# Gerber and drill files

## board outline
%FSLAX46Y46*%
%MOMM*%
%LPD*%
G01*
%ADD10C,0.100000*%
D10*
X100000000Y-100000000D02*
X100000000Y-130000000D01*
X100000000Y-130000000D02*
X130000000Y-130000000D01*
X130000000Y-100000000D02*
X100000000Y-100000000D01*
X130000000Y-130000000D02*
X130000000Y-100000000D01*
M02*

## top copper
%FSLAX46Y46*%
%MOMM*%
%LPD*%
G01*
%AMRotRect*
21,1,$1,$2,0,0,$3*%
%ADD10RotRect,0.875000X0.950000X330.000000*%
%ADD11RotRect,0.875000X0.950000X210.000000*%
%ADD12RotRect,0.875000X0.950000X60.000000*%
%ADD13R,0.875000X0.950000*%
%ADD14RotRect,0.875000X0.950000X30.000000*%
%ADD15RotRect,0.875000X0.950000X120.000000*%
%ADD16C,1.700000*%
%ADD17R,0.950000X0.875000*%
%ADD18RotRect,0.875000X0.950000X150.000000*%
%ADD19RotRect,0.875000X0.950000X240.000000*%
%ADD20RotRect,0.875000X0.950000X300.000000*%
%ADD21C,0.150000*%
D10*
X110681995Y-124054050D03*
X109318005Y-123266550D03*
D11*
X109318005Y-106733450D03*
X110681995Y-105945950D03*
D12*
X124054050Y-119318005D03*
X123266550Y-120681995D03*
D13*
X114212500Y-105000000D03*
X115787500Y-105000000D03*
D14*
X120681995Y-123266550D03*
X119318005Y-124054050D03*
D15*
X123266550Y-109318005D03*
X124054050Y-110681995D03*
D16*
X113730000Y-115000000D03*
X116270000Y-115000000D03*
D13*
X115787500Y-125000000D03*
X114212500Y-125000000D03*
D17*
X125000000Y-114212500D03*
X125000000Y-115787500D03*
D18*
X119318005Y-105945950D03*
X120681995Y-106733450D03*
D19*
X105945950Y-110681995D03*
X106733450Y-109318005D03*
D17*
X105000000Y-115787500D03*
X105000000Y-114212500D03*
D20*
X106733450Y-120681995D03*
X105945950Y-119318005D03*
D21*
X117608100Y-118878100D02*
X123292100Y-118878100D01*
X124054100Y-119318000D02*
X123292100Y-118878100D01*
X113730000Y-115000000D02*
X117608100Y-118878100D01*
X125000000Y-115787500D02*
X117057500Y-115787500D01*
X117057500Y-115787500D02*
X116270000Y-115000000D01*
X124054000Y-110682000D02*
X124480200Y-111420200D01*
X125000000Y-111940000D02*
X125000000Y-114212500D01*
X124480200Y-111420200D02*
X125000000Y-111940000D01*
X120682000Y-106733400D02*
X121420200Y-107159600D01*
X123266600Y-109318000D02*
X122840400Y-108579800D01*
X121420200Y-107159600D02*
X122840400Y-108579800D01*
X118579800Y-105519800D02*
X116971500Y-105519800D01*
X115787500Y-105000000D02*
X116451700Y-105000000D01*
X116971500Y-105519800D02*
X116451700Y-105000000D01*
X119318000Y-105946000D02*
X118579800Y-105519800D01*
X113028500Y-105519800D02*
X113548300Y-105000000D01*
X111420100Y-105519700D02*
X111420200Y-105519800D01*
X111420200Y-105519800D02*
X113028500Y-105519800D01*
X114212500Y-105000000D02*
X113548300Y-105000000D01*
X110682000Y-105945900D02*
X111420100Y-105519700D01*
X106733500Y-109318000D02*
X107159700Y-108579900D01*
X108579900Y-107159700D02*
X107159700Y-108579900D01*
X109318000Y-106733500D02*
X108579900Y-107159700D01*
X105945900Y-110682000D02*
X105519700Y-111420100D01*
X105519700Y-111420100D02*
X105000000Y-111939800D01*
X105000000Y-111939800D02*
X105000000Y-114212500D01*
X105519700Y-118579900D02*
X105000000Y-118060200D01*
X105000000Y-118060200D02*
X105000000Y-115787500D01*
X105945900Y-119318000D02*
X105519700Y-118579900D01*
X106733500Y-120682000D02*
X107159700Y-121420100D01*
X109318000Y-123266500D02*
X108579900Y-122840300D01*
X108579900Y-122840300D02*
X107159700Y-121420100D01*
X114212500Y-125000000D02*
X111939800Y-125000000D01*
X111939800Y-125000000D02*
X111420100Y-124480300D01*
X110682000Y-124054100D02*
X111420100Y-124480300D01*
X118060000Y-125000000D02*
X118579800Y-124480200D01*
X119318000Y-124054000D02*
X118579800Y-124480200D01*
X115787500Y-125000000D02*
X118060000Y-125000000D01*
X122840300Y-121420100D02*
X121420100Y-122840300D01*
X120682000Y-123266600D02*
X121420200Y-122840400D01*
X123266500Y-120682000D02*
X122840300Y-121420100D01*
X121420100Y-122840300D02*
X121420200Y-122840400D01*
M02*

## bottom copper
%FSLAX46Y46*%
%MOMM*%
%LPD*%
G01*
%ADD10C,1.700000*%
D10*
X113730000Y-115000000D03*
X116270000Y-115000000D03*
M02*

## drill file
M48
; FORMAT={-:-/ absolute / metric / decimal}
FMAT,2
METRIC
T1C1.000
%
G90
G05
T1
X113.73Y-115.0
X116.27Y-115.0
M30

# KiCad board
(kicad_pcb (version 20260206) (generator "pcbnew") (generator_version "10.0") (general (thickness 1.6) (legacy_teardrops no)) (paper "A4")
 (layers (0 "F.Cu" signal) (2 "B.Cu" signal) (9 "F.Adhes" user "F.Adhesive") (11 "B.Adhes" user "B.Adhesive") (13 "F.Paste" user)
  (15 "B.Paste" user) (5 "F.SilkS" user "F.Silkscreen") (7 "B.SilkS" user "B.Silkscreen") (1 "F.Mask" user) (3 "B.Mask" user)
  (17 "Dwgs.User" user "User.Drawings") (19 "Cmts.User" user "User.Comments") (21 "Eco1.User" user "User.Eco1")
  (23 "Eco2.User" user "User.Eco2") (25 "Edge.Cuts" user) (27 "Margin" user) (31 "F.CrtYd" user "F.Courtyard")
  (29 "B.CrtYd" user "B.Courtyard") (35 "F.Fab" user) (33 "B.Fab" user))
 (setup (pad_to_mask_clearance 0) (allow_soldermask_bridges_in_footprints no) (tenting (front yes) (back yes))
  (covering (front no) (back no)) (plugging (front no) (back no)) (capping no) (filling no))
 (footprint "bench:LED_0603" (layer "F.Cu") (at 110 123.6603 -30)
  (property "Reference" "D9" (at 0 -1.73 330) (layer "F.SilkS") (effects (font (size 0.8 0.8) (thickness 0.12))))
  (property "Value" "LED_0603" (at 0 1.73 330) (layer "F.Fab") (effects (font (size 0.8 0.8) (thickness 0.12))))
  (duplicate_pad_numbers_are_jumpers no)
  (pad "A" smd rect (at 0.7875 0 330) (size 0.875 0.95) (layers "F.Cu" "F.Mask" "F.Paste") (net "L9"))
  (pad "K" smd rect (at -0.7875 0 330) (size 0.875 0.95) (layers "F.Cu" "F.Mask" "F.Paste") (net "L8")))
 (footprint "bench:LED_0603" (layer "F.Cu") (at 110 106.3397 -150)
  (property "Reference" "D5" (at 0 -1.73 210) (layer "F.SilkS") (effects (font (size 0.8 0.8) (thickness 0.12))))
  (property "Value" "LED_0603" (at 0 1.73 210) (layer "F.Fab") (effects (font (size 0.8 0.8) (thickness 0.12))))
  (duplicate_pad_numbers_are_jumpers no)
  (pad "A" smd rect (at 0.7875 0 210) (size 0.875 0.95) (layers "F.Cu" "F.Mask" "F.Paste") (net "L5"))
  (pad "K" smd rect (at -0.7875 0 210) (size 0.875 0.95) (layers "F.Cu" "F.Mask" "F.Paste") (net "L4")))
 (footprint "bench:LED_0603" (layer "F.Cu") (at 123.6603 120 60)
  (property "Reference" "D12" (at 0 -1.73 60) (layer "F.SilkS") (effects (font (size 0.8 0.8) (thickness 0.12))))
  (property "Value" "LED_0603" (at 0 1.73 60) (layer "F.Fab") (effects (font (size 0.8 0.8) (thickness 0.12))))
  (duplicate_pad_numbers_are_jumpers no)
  (pad "A" smd rect (at 0.7875 0 60) (size 0.875 0.95) (layers "F.Cu" "F.Mask" "F.Paste") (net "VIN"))
  (pad "K" smd rect (at -0.7875 0 60) (size 0.875 0.95) (layers "F.Cu" "F.Mask" "F.Paste") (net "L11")))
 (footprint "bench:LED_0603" (layer "F.Cu") (at 115 105 180)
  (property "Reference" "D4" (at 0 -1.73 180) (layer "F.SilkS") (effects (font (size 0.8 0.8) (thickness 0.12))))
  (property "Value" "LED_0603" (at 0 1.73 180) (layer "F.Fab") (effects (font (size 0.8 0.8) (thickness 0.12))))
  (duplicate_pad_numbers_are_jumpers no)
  (pad "A" smd rect (at 0.7875 0 180) (size 0.875 0.95) (layers "F.Cu" "F.Mask" "F.Paste") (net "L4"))
  (pad "K" smd rect (at -0.7875 0 180) (size 0.875 0.95) (layers "F.Cu" "F.Mask" "F.Paste") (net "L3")))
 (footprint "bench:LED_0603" (layer "F.Cu") (at 120 123.6603 30)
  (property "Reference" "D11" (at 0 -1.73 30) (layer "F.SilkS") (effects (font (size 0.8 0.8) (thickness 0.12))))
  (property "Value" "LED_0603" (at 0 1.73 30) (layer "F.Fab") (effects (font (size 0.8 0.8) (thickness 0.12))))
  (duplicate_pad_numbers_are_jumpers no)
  (pad "A" smd rect (at 0.7875 0 30) (size 0.875 0.95) (layers "F.Cu" "F.Mask" "F.Paste") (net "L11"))
  (pad "K" smd rect (at -0.7875 0 30) (size 0.875 0.95) (layers "F.Cu" "F.Mask" "F.Paste") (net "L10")))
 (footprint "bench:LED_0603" (layer "F.Cu") (at 123.6603 110 120)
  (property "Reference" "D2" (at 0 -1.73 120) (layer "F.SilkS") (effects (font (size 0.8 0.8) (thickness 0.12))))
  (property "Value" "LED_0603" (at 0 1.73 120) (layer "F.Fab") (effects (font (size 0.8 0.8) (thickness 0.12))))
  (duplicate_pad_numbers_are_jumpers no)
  (pad "A" smd rect (at 0.7875 0 120) (size 0.875 0.95) (layers "F.Cu" "F.Mask" "F.Paste") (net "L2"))
  (pad "K" smd rect (at -0.7875 0 120) (size 0.875 0.95) (layers "F.Cu" "F.Mask" "F.Paste") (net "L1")))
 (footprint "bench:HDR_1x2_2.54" (layer "F.Cu") (at 113.73 115)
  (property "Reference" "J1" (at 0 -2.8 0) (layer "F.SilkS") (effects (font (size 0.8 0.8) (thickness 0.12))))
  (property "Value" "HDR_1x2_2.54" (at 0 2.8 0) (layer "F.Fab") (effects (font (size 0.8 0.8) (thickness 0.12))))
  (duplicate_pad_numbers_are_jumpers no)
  (pad "1" thru_hole circle (at 0 0) (size 1.7 1.7) (drill 1) (layers "*.Cu" "*.Mask") (remove_unused_layers no) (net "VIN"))
  (pad "2" thru_hole circle (at 2.54 0) (size 1.7 1.7) (drill 1) (layers "*.Cu" "*.Mask") (remove_unused_layers no) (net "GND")))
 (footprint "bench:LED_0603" (layer "F.Cu") (at 115 125)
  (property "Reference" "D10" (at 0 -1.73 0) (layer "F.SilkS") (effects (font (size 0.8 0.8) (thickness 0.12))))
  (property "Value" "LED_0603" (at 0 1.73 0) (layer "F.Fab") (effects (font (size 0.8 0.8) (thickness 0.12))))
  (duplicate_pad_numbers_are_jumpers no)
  (pad "A" smd rect (at 0.7875 0) (size 0.875 0.95) (layers "F.Cu" "F.Mask" "F.Paste") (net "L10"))
  (pad "K" smd rect (at -0.7875 0) (size 0.875 0.95) (layers "F.Cu" "F.Mask" "F.Paste") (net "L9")))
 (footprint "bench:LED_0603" (layer "F.Cu") (at 125 115 90)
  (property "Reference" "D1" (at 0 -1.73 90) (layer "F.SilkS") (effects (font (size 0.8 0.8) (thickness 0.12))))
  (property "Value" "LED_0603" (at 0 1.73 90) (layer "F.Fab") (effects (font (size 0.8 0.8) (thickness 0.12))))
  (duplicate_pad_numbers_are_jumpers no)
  (pad "A" smd rect (at 0.7875 0 90) (size 0.875 0.95) (layers "F.Cu" "F.Mask" "F.Paste") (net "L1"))
  (pad "K" smd rect (at -0.7875 0 90) (size 0.875 0.95) (layers "F.Cu" "F.Mask" "F.Paste") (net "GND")))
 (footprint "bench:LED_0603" (layer "F.Cu") (at 120 106.3397 150)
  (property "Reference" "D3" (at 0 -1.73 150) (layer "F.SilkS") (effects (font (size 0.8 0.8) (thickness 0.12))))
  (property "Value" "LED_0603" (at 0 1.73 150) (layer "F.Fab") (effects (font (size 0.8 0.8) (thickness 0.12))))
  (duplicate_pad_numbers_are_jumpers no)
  (pad "A" smd rect (at 0.7875 0 150) (size 0.875 0.95) (layers "F.Cu" "F.Mask" "F.Paste") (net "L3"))
  (pad "K" smd rect (at -0.7875 0 150) (size 0.875 0.95) (layers "F.Cu" "F.Mask" "F.Paste") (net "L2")))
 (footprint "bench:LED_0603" (layer "F.Cu") (at 106.3397 110 -120)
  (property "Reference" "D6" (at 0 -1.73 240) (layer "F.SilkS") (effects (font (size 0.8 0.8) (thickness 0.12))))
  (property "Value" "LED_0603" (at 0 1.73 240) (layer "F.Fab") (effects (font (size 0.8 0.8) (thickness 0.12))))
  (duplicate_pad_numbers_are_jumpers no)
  (pad "A" smd rect (at 0.7875 0 240) (size 0.875 0.95) (layers "F.Cu" "F.Mask" "F.Paste") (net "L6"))
  (pad "K" smd rect (at -0.7875 0 240) (size 0.875 0.95) (layers "F.Cu" "F.Mask" "F.Paste") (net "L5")))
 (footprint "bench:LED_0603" (layer "F.Cu") (at 105 115 -90)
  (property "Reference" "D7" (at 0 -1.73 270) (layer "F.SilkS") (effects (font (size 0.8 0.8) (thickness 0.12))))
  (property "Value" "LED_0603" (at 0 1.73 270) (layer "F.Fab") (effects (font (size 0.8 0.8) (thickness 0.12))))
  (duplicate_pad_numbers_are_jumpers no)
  (pad "A" smd rect (at 0.7875 0 270) (size 0.875 0.95) (layers "F.Cu" "F.Mask" "F.Paste") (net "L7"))
  (pad "K" smd rect (at -0.7875 0 270) (size 0.875 0.95) (layers "F.Cu" "F.Mask" "F.Paste") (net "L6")))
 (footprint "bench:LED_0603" (layer "F.Cu") (at 106.3397 120 -60)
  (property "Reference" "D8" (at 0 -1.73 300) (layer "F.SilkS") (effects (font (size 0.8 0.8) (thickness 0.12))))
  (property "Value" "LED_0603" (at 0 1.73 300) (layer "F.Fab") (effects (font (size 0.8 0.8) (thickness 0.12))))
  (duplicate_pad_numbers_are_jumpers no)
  (pad "A" smd rect (at 0.7875 0 300) (size 0.875 0.95) (layers "F.Cu" "F.Mask" "F.Paste") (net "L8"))
  (pad "K" smd rect (at -0.7875 0 300) (size 0.875 0.95) (layers "F.Cu" "F.Mask" "F.Paste") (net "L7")))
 (gr_line (start 100 100) (end 100 130) (stroke (width 0.1) (type solid)) (layer "Edge.Cuts"))
 (gr_line (start 100 130) (end 130 130) (stroke (width 0.1) (type solid)) (layer "Edge.Cuts"))
 (gr_line (start 130 100) (end 100 100) (stroke (width 0.1) (type solid)) (layer "Edge.Cuts"))
 (gr_line (start 130 130) (end 130 100) (stroke (width 0.1) (type solid)) (layer "Edge.Cuts"))
 (segment (start 117.6081 118.8781) (end 123.2921 118.8781) (width 0.15) (layer "F.Cu") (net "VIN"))
 (segment (start 124.0541 119.318) (end 123.2921 118.8781) (width 0.15) (layer "F.Cu") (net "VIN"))
 (segment (start 113.73 115) (end 117.6081 118.8781) (width 0.15) (layer "F.Cu") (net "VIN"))
 (segment (start 125 115.7875) (end 117.0575 115.7875) (width 0.15) (layer "F.Cu") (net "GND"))
 (segment (start 117.0575 115.7875) (end 116.27 115) (width 0.15) (layer "F.Cu") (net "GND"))
 (segment (start 124.054 110.682) (end 124.4802 111.4202) (width 0.15) (layer "F.Cu") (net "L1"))
 (segment (start 125 111.94) (end 125 114.2125) (width 0.15) (layer "F.Cu") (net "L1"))
 (segment (start 124.4802 111.4202) (end 125 111.94) (width 0.15) (layer "F.Cu") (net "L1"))
 (segment (start 120.682 106.7334) (end 121.4202 107.1596) (width 0.15) (layer "F.Cu") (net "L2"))
 (segment (start 123.2666 109.318) (end 122.8404 108.5798) (width 0.15) (layer "F.Cu") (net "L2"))
 (segment (start 121.4202 107.1596) (end 122.8404 108.5798) (width 0.15) (layer "F.Cu") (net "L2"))
 (segment (start 118.5798 105.5198) (end 116.9715 105.5198) (width 0.15) (layer "F.Cu") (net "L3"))
 (segment (start 115.7875 105) (end 116.4517 105) (width 0.15) (layer "F.Cu") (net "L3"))
 (segment (start 116.9715 105.5198) (end 116.4517 105) (width 0.15) (layer "F.Cu") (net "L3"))
 (segment (start 119.318 105.946) (end 118.5798 105.5198) (width 0.15) (layer "F.Cu") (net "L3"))
 (segment (start 113.0285 105.5198) (end 113.5483 105) (width 0.15) (layer "F.Cu") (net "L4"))
 (segment (start 111.4201 105.5197) (end 111.4202 105.5198) (width 0.15) (layer "F.Cu") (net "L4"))
 (segment (start 111.4202 105.5198) (end 113.0285 105.5198) (width 0.15) (layer "F.Cu") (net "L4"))
 (segment (start 114.2125 105) (end 113.5483 105) (width 0.15) (layer "F.Cu") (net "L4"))
 (segment (start 110.682 105.9459) (end 111.4201 105.5197) (width 0.15) (layer "F.Cu") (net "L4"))
 (segment (start 106.7335 109.318) (end 107.1597 108.5799) (width 0.15) (layer "F.Cu") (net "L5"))
 (segment (start 108.5799 107.1597) (end 107.1597 108.5799) (width 0.15) (layer "F.Cu") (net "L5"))
 (segment (start 109.318 106.7335) (end 108.5799 107.1597) (width 0.15) (layer "F.Cu") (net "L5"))
 (segment (start 105.9459 110.682) (end 105.5197 111.4201) (width 0.15) (layer "F.Cu") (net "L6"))
 (segment (start 105.5197 111.4201) (end 105 111.9398) (width 0.15) (layer "F.Cu") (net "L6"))
 (segment (start 105 111.9398) (end 105 114.2125) (width 0.15) (layer "F.Cu") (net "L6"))
 (segment (start 105.5197 118.5799) (end 105 118.0602) (width 0.15) (layer "F.Cu") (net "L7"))
 (segment (start 105 118.0602) (end 105 115.7875) (width 0.15) (layer "F.Cu") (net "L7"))
 (segment (start 105.9459 119.318) (end 105.5197 118.5799) (width 0.15) (layer "F.Cu") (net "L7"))
 (segment (start 106.7335 120.682) (end 107.1597 121.4201) (width 0.15) (layer "F.Cu") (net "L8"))
 (segment (start 109.318 123.2665) (end 108.5799 122.8403) (width 0.15) (layer "F.Cu") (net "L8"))
 (segment (start 108.5799 122.8403) (end 107.1597 121.4201) (width 0.15) (layer "F.Cu") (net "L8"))
 (segment (start 114.2125 125) (end 111.9398 125) (width 0.15) (layer "F.Cu") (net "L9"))
 (segment (start 111.9398 125) (end 111.4201 124.4803) (width 0.15) (layer "F.Cu") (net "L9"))
 (segment (start 110.682 124.0541) (end 111.4201 124.4803) (width 0.15) (layer "F.Cu") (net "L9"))
 (segment (start 118.06 125) (end 118.5798 124.4802) (width 0.15) (layer "F.Cu") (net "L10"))
 (segment (start 119.318 124.054) (end 118.5798 124.4802) (width 0.15) (layer "F.Cu") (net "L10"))
 (segment (start 115.7875 125) (end 118.06 125) (width 0.15) (layer "F.Cu") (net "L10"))
 (segment (start 122.8403 121.4201) (end 121.4201 122.8403) (width 0.15) (layer "F.Cu") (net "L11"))
 (segment (start 120.682 123.2666) (end 121.4202 122.8404) (width 0.15) (layer "F.Cu") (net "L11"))
 (segment (start 123.2665 120.682) (end 122.8403 121.4201) (width 0.15) (layer "F.Cu") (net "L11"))
 (segment (start 121.4201 122.8403) (end 121.4202 122.8404) (width 0.15) (layer "F.Cu") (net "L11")))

